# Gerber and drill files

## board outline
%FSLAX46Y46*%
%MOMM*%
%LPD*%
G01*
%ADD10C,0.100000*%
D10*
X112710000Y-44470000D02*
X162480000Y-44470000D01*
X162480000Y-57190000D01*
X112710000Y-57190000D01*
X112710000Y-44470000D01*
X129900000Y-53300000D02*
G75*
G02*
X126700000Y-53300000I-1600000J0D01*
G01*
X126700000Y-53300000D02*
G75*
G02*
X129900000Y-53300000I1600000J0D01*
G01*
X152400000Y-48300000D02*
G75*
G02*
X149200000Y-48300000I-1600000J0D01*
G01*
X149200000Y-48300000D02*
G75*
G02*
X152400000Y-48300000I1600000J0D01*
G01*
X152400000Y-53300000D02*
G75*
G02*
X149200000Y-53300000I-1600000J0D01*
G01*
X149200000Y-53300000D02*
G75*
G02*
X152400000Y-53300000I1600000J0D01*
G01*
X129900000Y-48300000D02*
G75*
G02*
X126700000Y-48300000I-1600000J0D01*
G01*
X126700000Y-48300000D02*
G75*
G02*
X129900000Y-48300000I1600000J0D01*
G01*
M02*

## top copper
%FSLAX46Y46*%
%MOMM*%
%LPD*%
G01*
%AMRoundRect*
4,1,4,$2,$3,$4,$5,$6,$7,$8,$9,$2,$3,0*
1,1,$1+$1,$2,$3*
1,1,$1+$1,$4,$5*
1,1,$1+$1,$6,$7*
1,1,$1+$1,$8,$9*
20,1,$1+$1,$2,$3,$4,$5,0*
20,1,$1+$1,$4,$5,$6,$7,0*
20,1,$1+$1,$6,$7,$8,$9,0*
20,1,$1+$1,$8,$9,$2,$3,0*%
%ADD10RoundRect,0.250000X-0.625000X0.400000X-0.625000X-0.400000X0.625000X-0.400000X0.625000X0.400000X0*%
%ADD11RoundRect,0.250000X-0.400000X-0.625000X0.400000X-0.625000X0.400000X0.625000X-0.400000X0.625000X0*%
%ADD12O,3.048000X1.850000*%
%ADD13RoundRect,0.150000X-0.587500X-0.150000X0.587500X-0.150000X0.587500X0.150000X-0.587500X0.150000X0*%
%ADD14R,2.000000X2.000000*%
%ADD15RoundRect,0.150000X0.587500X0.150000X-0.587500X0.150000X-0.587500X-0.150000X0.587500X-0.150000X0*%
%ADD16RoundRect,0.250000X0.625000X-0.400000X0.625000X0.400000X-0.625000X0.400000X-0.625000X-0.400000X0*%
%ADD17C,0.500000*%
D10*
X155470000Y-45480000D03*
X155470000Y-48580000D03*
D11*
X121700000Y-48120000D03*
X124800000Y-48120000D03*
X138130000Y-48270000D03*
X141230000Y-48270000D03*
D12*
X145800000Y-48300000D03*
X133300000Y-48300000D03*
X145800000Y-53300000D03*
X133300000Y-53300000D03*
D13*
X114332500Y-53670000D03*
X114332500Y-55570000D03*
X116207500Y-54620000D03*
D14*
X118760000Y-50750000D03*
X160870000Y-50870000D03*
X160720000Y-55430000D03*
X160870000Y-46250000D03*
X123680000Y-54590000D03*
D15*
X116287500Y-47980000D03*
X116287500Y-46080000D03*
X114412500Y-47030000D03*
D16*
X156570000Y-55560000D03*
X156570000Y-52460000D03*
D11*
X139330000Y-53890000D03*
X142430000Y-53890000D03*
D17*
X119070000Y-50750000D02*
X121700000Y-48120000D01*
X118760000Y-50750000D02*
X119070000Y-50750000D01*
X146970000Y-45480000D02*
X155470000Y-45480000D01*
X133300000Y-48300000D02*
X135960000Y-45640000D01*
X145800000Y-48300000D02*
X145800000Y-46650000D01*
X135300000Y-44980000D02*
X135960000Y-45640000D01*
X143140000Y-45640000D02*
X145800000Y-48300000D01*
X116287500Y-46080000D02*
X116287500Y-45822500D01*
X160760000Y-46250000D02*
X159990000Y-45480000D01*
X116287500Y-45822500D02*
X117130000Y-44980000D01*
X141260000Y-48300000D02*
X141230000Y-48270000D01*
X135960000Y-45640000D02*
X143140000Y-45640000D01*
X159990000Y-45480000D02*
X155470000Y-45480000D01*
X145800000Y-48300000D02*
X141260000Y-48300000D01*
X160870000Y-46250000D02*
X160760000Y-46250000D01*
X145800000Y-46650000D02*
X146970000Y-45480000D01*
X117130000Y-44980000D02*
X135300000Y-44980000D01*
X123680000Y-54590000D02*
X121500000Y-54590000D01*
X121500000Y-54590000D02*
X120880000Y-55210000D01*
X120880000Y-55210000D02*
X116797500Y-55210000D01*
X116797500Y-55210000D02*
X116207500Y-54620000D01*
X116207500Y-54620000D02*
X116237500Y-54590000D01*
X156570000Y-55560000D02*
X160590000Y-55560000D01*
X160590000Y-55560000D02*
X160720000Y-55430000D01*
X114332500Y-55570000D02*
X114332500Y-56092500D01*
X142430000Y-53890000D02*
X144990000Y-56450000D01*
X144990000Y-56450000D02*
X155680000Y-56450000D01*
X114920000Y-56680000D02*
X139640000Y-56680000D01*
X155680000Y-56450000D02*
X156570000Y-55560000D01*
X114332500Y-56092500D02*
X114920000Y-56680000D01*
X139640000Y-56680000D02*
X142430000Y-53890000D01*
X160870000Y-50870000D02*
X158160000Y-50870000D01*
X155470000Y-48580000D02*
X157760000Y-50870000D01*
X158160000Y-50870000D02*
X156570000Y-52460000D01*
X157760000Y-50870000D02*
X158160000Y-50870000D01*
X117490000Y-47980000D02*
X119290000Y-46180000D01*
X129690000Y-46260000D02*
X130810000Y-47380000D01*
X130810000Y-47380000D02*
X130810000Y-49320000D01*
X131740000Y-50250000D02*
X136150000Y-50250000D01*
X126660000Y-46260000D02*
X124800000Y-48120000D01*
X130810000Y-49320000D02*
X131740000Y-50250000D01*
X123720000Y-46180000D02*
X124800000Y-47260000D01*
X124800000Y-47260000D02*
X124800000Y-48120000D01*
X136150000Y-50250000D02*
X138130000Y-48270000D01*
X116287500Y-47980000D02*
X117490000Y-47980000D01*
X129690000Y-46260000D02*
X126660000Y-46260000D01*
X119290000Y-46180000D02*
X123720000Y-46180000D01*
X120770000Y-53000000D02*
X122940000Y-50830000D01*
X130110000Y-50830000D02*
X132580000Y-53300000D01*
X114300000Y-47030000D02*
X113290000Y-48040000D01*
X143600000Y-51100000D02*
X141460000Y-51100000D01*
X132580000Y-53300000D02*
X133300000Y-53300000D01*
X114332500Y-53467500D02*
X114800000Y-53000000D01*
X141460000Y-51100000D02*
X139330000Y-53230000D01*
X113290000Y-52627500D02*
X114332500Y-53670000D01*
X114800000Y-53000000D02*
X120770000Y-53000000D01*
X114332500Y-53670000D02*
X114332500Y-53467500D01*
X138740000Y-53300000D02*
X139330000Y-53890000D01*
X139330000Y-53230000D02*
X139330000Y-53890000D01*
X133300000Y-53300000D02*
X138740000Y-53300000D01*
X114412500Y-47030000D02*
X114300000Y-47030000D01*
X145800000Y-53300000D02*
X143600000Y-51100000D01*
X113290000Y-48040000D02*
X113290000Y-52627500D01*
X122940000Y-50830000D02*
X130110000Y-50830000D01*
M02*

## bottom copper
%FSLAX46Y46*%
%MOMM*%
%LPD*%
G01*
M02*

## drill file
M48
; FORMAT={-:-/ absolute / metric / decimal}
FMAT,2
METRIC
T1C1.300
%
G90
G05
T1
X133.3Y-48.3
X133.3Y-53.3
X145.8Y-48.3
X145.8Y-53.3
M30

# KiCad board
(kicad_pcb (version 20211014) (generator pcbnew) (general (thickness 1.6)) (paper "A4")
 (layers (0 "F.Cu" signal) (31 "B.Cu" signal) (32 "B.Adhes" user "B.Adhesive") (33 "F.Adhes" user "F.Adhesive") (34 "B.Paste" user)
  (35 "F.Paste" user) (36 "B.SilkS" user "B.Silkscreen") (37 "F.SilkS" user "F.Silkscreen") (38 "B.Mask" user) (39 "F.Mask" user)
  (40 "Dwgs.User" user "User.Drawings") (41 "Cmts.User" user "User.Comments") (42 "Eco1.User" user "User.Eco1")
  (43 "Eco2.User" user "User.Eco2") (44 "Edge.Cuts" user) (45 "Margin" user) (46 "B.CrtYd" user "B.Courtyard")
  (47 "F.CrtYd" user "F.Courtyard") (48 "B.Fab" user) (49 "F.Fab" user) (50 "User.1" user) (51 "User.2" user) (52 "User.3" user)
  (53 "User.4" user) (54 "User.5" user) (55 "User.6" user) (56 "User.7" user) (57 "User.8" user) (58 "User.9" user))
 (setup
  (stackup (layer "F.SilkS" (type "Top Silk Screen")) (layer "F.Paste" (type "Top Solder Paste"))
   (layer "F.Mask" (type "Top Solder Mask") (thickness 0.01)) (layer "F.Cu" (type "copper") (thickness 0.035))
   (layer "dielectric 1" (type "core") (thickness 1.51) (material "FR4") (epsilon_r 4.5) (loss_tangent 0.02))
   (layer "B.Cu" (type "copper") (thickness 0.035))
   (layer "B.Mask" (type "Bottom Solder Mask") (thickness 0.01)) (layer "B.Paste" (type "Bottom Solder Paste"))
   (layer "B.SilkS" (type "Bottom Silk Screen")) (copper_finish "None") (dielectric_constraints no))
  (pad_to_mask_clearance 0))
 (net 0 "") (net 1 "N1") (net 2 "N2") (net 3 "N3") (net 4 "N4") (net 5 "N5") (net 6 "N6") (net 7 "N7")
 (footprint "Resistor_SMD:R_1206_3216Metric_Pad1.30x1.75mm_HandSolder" (layer "F.Cu") (at 155.47 47.03 -90)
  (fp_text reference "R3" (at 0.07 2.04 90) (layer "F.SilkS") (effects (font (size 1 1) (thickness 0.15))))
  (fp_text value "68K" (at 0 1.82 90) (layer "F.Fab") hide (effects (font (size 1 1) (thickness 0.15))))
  (pad "1" smd roundrect (at -1.55 0 270) (size 1.3 1.75) (layers "F.Cu" "F.Paste" "F.Mask") (roundrect_rratio 0.1923076923) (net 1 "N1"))
  (pad "2" smd roundrect (at 1.55 0 270) (size 1.3 1.75) (layers "F.Cu" "F.Paste" "F.Mask") (roundrect_rratio 0.1923076923) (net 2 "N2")))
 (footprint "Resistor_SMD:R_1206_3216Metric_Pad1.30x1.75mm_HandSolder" (layer "F.Cu") (at 123.25 48.12)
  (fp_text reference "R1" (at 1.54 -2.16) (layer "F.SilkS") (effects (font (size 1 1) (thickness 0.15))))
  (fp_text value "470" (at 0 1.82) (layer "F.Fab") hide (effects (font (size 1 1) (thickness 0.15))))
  (pad "1" smd roundrect (at -1.55 0) (size 1.3 1.75) (layers "F.Cu" "F.Paste" "F.Mask") (roundrect_rratio 0.1923076923) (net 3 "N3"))
  (pad "2" smd roundrect (at 1.55 0) (size 1.3 1.75) (layers "F.Cu" "F.Paste" "F.Mask") (roundrect_rratio 0.1923076923) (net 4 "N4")))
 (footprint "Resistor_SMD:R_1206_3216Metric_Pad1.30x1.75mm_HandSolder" (layer "F.Cu") (at 139.68 48.27)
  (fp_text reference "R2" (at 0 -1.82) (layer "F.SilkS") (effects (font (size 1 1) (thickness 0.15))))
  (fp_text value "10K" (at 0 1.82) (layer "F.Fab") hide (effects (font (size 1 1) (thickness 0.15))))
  (pad "1" smd roundrect (at -1.55 0) (size 1.3 1.75) (layers "F.Cu" "F.Paste" "F.Mask") (roundrect_rratio 0.1923076923) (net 4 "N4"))
  (pad "2" smd roundrect (at 1.55 0) (size 1.3 1.75) (layers "F.Cu" "F.Paste" "F.Mask") (roundrect_rratio 0.1923076923) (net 1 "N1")))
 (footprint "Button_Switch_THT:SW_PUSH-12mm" (layer "F.Cu") (at 133.3 48.3)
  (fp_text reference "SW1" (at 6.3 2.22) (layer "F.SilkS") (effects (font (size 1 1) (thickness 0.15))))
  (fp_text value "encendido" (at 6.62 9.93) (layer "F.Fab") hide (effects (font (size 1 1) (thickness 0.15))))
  (pad "1" thru_hole oval (at 12.5 0) (size 3.048 1.85) (drill 1.3) (layers *.Cu "F.Mask") (remove_unused_layers) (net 1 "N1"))
  (pad "1" thru_hole oval (at 0 0) (size 3.048 1.85) (drill 1.3) (layers *.Cu "F.Mask") (remove_unused_layers) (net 1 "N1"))
  (pad "2" thru_hole oval (at 12.5 5) (size 3.048 1.85) (drill 1.3) (layers *.Cu "F.Mask") (remove_unused_layers) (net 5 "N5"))
  (pad "2" thru_hole oval (at 0 5) (size 3.048 1.85) (drill 1.3) (layers *.Cu "F.Mask") (remove_unused_layers) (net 5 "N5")))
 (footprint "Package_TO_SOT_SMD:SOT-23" (layer "F.Cu") (at 115.27 54.62)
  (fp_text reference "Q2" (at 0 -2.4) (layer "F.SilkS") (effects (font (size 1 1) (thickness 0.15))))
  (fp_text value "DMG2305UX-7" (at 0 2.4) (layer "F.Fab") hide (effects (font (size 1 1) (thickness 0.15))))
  (pad "1" smd roundrect (at -0.9375 -0.95) (size 1.475 0.6) (layers "F.Cu" "F.Paste" "F.Mask") (roundrect_rratio 0.25) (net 5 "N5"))
  (pad "2" smd roundrect (at -0.9375 0.95) (size 1.475 0.6) (layers "F.Cu" "F.Paste" "F.Mask") (roundrect_rratio 0.25) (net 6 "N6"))
  (pad "3" smd roundrect (at 0.9375 0) (size 1.475 0.6) (layers "F.Cu" "F.Paste" "F.Mask") (roundrect_rratio 0.25) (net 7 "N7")))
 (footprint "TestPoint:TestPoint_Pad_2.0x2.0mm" (layer "F.Cu") (at 118.76 50.75)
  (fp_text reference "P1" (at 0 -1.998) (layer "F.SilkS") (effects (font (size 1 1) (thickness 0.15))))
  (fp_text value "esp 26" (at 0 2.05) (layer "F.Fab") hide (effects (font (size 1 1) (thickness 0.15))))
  (pad "1" smd rect (at 0 0) (size 2 2) (layers "F.Cu" "F.Mask") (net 3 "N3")))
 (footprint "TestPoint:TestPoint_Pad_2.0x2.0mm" (layer "F.Cu") (at 160.87 50.87)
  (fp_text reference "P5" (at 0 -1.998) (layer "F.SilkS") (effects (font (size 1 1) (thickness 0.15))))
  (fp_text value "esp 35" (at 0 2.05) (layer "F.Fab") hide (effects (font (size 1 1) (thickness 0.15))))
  (pad "1" smd rect (at 0 0) (size 2 2) (layers "F.Cu" "F.Mask") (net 2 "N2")))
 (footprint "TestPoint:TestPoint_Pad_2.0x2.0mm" (layer "F.Cu") (at 160.72 55.43)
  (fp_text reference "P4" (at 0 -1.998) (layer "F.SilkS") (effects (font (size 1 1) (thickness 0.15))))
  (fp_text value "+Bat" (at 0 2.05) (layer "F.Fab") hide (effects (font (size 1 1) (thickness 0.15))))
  (pad "1" smd rect (at 0 0) (size 2 2) (layers "F.Cu" "F.Mask") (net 6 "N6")))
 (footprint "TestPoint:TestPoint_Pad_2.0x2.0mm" (layer "F.Cu") (at 160.87 46.25)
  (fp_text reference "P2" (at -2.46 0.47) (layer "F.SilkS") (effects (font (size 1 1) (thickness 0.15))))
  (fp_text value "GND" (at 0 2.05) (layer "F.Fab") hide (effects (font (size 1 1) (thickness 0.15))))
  (pad "1" smd rect (at 0 0) (size 2 2) (layers "F.Cu" "F.Mask") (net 1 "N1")))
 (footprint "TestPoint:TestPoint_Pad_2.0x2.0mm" (layer "F.Cu") (at 123.68 54.59)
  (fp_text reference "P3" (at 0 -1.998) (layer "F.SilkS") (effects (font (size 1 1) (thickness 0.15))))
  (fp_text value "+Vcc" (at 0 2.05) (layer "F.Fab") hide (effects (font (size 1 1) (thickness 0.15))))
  (pad "1" smd rect (at 0 0) (size 2 2) (layers "F.Cu" "F.Mask") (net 7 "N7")))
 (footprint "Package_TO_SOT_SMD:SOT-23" (layer "F.Cu") (at 115.35 47.03 180)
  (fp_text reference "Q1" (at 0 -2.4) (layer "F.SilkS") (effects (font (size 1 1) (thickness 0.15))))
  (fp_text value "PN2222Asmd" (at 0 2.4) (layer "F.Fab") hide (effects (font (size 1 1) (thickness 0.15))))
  (pad "1" smd roundrect (at -0.9375 -0.95 180) (size 1.475 0.6) (layers "F.Cu" "F.Paste" "F.Mask") (roundrect_rratio 0.25) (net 4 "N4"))
  (pad "2" smd roundrect (at -0.9375 0.95 180) (size 1.475 0.6) (layers "F.Cu" "F.Paste" "F.Mask") (roundrect_rratio 0.25) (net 1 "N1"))
  (pad "3" smd roundrect (at 0.9375 0 180) (size 1.475 0.6) (layers "F.Cu" "F.Paste" "F.Mask") (roundrect_rratio 0.25) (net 5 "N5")))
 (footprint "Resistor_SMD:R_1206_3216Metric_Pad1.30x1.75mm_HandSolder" (layer "F.Cu") (at 156.57 54.01 90)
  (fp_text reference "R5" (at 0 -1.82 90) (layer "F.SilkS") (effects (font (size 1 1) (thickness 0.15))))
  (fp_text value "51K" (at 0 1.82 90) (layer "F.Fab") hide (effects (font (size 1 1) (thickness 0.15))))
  (pad "1" smd roundrect (at -1.55 0 90) (size 1.3 1.75) (layers "F.Cu" "F.Paste" "F.Mask") (roundrect_rratio 0.1923076923) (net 6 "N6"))
  (pad "2" smd roundrect (at 1.55 0 90) (size 1.3 1.75) (layers "F.Cu" "F.Paste" "F.Mask") (roundrect_rratio 0.1923076923) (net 2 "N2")))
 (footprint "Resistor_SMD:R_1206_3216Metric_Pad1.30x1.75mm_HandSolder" (layer "F.Cu") (at 140.88 53.89)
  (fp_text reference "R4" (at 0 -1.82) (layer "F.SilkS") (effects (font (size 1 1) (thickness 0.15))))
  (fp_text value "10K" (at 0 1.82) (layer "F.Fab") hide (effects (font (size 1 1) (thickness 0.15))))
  (pad "1" smd roundrect (at -1.55 0) (size 1.3 1.75) (layers "F.Cu" "F.Paste" "F.Mask") (roundrect_rratio 0.1923076923) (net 5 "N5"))
  (pad "2" smd roundrect (at 1.55 0) (size 1.3 1.75) (layers "F.Cu" "F.Paste" "F.Mask") (roundrect_rratio 0.1923076923) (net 6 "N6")))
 (gr_rect (start 162.48 57.19) (end 112.71 44.47) (layer "Edge.Cuts") (width 0.1) (fill none))
 (gr_circle (center 128.3 53.3) (end 129.9 53.3) (layer "Edge.Cuts") (width 0.1) (fill none))
 (gr_circle (center 150.8 48.3) (end 152.4 48.3) (layer "Edge.Cuts") (width 0.1) (fill none))
 (gr_circle (center 150.8 53.3) (end 152.4 53.3) (layer "Edge.Cuts") (width 0.1) (fill none))
 (gr_circle (center 128.3 48.3) (end 129.9 48.3) (layer "Edge.Cuts") (width 0.1) (fill none))
 (segment (start 119.07 50.75) (end 121.7 48.12) (width 0.5) (layer "F.Cu") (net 3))
 (segment (start 118.76 50.75) (end 119.07 50.75) (width 0.5) (layer "F.Cu") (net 3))
 (segment (start 146.97 45.48) (end 155.47 45.48) (width 0.5) (layer "F.Cu") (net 1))
 (segment (start 133.3 48.3) (end 135.96 45.64) (width 0.5) (layer "F.Cu") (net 1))
 (segment (start 145.8 48.3) (end 145.8 46.65) (width 0.5) (layer "F.Cu") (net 1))
 (segment (start 135.3 44.98) (end 135.96 45.64) (width 0.5) (layer "F.Cu") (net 1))
 (segment (start 143.14 45.64) (end 145.8 48.3) (width 0.5) (layer "F.Cu") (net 1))
 (segment (start 116.2875 46.08) (end 116.2875 45.8225) (width 0.5) (layer "F.Cu") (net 1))
 (segment (start 160.76 46.25) (end 159.99 45.48) (width 0.5) (layer "F.Cu") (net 1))
 (segment (start 116.2875 45.8225) (end 117.13 44.98) (width 0.5) (layer "F.Cu") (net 1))
 (segment (start 141.26 48.3) (end 141.23 48.27) (width 0.5) (layer "F.Cu") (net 1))
 (segment (start 135.96 45.64) (end 143.14 45.64) (width 0.5) (layer "F.Cu") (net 1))
 (segment (start 159.99 45.48) (end 155.47 45.48) (width 0.5) (layer "F.Cu") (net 1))
 (segment (start 145.8 48.3) (end 141.26 48.3) (width 0.5) (layer "F.Cu") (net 1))
 (segment (start 160.87 46.25) (end 160.76 46.25) (width 0.5) (layer "F.Cu") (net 1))
 (segment (start 145.8 46.65) (end 146.97 45.48) (width 0.5) (layer "F.Cu") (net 1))
 (segment (start 117.13 44.98) (end 135.3 44.98) (width 0.5) (layer "F.Cu") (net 1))
 (segment (start 123.68 54.59) (end 121.5 54.59) (width 0.5) (layer "F.Cu") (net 7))
 (segment (start 121.5 54.59) (end 120.88 55.21) (width 0.5) (layer "F.Cu") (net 7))
 (segment (start 120.88 55.21) (end 116.7975 55.21) (width 0.5) (layer "F.Cu") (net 7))
 (segment (start 116.7975 55.21) (end 116.2075 54.62) (width 0.5) (layer "F.Cu") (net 7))
 (segment (start 116.2075 54.62) (end 116.2375 54.59) (width 0.5) (layer "F.Cu") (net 7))
 (segment (start 156.57 55.56) (end 160.59 55.56) (width 0.5) (layer "F.Cu") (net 6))
 (segment (start 160.59 55.56) (end 160.72 55.43) (width 0.5) (layer "F.Cu") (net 6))
 (segment (start 114.3325 55.57) (end 114.3325 56.0925) (width 0.5) (layer "F.Cu") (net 6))
 (segment (start 142.43 53.89) (end 144.99 56.45) (width 0.5) (layer "F.Cu") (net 6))
 (segment (start 144.99 56.45) (end 155.68 56.45) (width 0.5) (layer "F.Cu") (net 6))
 (segment (start 114.92 56.68) (end 139.64 56.68) (width 0.5) (layer "F.Cu") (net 6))
 (segment (start 155.68 56.45) (end 156.57 55.56) (width 0.5) (layer "F.Cu") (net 6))
 (segment (start 114.3325 56.0925) (end 114.92 56.68) (width 0.5) (layer "F.Cu") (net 6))
 (segment (start 139.64 56.68) (end 142.43 53.89) (width 0.5) (layer "F.Cu") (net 6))
 (segment (start 160.87 50.87) (end 158.16 50.87) (width 0.5) (layer "F.Cu") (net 2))
 (segment (start 155.47 48.58) (end 157.76 50.87) (width 0.5) (layer "F.Cu") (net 2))
 (segment (start 158.16 50.87) (end 156.57 52.46) (width 0.5) (layer "F.Cu") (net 2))
 (segment (start 157.76 50.87) (end 158.16 50.87) (width 0.5) (layer "F.Cu") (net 2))
 (segment (start 117.49 47.98) (end 119.29 46.18) (width 0.5) (layer "F.Cu") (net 4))
 (segment (start 129.69 46.26) (end 130.81 47.38) (width 0.5) (layer "F.Cu") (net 4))
 (segment (start 130.81 47.38) (end 130.81 49.32) (width 0.5) (layer "F.Cu") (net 4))
 (segment (start 131.74 50.25) (end 136.15 50.25) (width 0.5) (layer "F.Cu") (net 4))
 (segment (start 126.66 46.26) (end 124.8 48.12) (width 0.5) (layer "F.Cu") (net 4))
 (segment (start 130.81 49.32) (end 131.74 50.25) (width 0.5) (layer "F.Cu") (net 4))
 (segment (start 123.72 46.18) (end 124.8 47.26) (width 0.5) (layer "F.Cu") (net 4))
 (segment (start 124.8 47.26) (end 124.8 48.12) (width 0.5) (layer "F.Cu") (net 4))
 (segment (start 136.15 50.25) (end 138.13 48.27) (width 0.5) (layer "F.Cu") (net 4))
 (segment (start 116.2875 47.98) (end 117.49 47.98) (width 0.5) (layer "F.Cu") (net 4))
 (segment (start 129.69 46.26) (end 126.66 46.26) (width 0.5) (layer "F.Cu") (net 4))
 (segment (start 119.29 46.18) (end 123.72 46.18) (width 0.5) (layer "F.Cu") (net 4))
 (segment (start 120.77 53) (end 122.94 50.83) (width 0.5) (layer "F.Cu") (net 5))
 (segment (start 130.11 50.83) (end 132.58 53.3) (width 0.5) (layer "F.Cu") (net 5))
 (segment (start 114.3 47.03) (end 113.29 48.04) (width 0.5) (layer "F.Cu") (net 5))
 (segment (start 143.6 51.1) (end 141.46 51.1) (width 0.5) (layer "F.Cu") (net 5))
 (segment (start 132.58 53.3) (end 133.3 53.3) (width 0.5) (layer "F.Cu") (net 5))
 (segment (start 114.3325 53.4675) (end 114.8 53) (width 0.5) (layer "F.Cu") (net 5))
 (segment (start 141.46 51.1) (end 139.33 53.23) (width 0.5) (layer "F.Cu") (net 5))
 (segment (start 113.29 52.6275) (end 114.3325 53.67) (width 0.5) (layer "F.Cu") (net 5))
 (segment (start 114.8 53) (end 120.77 53) (width 0.5) (layer "F.Cu") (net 5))
 (segment (start 114.3325 53.67) (end 114.3325 53.4675) (width 0.5) (layer "F.Cu") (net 5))
 (segment (start 138.74 53.3) (end 139.33 53.89) (width 0.5) (layer "F.Cu") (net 5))
 (segment (start 139.33 53.23) (end 139.33 53.89) (width 0.5) (layer "F.Cu") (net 5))
 (segment (start 133.3 53.3) (end 138.74 53.3) (width 0.5) (layer "F.Cu") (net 5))
 (segment (start 114.4125 47.03) (end 114.3 47.03) (width 0.5) (layer "F.Cu") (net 5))
 (segment (start 145.8 53.3) (end 143.6 51.1) (width 0.5) (layer "F.Cu") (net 5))
 (segment (start 113.29 48.04) (end 113.29 52.6275) (width 0.5) (layer "F.Cu") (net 5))
 (segment (start 122.94 50.83) (end 130.11 50.83) (width 0.5) (layer "F.Cu") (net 5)))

